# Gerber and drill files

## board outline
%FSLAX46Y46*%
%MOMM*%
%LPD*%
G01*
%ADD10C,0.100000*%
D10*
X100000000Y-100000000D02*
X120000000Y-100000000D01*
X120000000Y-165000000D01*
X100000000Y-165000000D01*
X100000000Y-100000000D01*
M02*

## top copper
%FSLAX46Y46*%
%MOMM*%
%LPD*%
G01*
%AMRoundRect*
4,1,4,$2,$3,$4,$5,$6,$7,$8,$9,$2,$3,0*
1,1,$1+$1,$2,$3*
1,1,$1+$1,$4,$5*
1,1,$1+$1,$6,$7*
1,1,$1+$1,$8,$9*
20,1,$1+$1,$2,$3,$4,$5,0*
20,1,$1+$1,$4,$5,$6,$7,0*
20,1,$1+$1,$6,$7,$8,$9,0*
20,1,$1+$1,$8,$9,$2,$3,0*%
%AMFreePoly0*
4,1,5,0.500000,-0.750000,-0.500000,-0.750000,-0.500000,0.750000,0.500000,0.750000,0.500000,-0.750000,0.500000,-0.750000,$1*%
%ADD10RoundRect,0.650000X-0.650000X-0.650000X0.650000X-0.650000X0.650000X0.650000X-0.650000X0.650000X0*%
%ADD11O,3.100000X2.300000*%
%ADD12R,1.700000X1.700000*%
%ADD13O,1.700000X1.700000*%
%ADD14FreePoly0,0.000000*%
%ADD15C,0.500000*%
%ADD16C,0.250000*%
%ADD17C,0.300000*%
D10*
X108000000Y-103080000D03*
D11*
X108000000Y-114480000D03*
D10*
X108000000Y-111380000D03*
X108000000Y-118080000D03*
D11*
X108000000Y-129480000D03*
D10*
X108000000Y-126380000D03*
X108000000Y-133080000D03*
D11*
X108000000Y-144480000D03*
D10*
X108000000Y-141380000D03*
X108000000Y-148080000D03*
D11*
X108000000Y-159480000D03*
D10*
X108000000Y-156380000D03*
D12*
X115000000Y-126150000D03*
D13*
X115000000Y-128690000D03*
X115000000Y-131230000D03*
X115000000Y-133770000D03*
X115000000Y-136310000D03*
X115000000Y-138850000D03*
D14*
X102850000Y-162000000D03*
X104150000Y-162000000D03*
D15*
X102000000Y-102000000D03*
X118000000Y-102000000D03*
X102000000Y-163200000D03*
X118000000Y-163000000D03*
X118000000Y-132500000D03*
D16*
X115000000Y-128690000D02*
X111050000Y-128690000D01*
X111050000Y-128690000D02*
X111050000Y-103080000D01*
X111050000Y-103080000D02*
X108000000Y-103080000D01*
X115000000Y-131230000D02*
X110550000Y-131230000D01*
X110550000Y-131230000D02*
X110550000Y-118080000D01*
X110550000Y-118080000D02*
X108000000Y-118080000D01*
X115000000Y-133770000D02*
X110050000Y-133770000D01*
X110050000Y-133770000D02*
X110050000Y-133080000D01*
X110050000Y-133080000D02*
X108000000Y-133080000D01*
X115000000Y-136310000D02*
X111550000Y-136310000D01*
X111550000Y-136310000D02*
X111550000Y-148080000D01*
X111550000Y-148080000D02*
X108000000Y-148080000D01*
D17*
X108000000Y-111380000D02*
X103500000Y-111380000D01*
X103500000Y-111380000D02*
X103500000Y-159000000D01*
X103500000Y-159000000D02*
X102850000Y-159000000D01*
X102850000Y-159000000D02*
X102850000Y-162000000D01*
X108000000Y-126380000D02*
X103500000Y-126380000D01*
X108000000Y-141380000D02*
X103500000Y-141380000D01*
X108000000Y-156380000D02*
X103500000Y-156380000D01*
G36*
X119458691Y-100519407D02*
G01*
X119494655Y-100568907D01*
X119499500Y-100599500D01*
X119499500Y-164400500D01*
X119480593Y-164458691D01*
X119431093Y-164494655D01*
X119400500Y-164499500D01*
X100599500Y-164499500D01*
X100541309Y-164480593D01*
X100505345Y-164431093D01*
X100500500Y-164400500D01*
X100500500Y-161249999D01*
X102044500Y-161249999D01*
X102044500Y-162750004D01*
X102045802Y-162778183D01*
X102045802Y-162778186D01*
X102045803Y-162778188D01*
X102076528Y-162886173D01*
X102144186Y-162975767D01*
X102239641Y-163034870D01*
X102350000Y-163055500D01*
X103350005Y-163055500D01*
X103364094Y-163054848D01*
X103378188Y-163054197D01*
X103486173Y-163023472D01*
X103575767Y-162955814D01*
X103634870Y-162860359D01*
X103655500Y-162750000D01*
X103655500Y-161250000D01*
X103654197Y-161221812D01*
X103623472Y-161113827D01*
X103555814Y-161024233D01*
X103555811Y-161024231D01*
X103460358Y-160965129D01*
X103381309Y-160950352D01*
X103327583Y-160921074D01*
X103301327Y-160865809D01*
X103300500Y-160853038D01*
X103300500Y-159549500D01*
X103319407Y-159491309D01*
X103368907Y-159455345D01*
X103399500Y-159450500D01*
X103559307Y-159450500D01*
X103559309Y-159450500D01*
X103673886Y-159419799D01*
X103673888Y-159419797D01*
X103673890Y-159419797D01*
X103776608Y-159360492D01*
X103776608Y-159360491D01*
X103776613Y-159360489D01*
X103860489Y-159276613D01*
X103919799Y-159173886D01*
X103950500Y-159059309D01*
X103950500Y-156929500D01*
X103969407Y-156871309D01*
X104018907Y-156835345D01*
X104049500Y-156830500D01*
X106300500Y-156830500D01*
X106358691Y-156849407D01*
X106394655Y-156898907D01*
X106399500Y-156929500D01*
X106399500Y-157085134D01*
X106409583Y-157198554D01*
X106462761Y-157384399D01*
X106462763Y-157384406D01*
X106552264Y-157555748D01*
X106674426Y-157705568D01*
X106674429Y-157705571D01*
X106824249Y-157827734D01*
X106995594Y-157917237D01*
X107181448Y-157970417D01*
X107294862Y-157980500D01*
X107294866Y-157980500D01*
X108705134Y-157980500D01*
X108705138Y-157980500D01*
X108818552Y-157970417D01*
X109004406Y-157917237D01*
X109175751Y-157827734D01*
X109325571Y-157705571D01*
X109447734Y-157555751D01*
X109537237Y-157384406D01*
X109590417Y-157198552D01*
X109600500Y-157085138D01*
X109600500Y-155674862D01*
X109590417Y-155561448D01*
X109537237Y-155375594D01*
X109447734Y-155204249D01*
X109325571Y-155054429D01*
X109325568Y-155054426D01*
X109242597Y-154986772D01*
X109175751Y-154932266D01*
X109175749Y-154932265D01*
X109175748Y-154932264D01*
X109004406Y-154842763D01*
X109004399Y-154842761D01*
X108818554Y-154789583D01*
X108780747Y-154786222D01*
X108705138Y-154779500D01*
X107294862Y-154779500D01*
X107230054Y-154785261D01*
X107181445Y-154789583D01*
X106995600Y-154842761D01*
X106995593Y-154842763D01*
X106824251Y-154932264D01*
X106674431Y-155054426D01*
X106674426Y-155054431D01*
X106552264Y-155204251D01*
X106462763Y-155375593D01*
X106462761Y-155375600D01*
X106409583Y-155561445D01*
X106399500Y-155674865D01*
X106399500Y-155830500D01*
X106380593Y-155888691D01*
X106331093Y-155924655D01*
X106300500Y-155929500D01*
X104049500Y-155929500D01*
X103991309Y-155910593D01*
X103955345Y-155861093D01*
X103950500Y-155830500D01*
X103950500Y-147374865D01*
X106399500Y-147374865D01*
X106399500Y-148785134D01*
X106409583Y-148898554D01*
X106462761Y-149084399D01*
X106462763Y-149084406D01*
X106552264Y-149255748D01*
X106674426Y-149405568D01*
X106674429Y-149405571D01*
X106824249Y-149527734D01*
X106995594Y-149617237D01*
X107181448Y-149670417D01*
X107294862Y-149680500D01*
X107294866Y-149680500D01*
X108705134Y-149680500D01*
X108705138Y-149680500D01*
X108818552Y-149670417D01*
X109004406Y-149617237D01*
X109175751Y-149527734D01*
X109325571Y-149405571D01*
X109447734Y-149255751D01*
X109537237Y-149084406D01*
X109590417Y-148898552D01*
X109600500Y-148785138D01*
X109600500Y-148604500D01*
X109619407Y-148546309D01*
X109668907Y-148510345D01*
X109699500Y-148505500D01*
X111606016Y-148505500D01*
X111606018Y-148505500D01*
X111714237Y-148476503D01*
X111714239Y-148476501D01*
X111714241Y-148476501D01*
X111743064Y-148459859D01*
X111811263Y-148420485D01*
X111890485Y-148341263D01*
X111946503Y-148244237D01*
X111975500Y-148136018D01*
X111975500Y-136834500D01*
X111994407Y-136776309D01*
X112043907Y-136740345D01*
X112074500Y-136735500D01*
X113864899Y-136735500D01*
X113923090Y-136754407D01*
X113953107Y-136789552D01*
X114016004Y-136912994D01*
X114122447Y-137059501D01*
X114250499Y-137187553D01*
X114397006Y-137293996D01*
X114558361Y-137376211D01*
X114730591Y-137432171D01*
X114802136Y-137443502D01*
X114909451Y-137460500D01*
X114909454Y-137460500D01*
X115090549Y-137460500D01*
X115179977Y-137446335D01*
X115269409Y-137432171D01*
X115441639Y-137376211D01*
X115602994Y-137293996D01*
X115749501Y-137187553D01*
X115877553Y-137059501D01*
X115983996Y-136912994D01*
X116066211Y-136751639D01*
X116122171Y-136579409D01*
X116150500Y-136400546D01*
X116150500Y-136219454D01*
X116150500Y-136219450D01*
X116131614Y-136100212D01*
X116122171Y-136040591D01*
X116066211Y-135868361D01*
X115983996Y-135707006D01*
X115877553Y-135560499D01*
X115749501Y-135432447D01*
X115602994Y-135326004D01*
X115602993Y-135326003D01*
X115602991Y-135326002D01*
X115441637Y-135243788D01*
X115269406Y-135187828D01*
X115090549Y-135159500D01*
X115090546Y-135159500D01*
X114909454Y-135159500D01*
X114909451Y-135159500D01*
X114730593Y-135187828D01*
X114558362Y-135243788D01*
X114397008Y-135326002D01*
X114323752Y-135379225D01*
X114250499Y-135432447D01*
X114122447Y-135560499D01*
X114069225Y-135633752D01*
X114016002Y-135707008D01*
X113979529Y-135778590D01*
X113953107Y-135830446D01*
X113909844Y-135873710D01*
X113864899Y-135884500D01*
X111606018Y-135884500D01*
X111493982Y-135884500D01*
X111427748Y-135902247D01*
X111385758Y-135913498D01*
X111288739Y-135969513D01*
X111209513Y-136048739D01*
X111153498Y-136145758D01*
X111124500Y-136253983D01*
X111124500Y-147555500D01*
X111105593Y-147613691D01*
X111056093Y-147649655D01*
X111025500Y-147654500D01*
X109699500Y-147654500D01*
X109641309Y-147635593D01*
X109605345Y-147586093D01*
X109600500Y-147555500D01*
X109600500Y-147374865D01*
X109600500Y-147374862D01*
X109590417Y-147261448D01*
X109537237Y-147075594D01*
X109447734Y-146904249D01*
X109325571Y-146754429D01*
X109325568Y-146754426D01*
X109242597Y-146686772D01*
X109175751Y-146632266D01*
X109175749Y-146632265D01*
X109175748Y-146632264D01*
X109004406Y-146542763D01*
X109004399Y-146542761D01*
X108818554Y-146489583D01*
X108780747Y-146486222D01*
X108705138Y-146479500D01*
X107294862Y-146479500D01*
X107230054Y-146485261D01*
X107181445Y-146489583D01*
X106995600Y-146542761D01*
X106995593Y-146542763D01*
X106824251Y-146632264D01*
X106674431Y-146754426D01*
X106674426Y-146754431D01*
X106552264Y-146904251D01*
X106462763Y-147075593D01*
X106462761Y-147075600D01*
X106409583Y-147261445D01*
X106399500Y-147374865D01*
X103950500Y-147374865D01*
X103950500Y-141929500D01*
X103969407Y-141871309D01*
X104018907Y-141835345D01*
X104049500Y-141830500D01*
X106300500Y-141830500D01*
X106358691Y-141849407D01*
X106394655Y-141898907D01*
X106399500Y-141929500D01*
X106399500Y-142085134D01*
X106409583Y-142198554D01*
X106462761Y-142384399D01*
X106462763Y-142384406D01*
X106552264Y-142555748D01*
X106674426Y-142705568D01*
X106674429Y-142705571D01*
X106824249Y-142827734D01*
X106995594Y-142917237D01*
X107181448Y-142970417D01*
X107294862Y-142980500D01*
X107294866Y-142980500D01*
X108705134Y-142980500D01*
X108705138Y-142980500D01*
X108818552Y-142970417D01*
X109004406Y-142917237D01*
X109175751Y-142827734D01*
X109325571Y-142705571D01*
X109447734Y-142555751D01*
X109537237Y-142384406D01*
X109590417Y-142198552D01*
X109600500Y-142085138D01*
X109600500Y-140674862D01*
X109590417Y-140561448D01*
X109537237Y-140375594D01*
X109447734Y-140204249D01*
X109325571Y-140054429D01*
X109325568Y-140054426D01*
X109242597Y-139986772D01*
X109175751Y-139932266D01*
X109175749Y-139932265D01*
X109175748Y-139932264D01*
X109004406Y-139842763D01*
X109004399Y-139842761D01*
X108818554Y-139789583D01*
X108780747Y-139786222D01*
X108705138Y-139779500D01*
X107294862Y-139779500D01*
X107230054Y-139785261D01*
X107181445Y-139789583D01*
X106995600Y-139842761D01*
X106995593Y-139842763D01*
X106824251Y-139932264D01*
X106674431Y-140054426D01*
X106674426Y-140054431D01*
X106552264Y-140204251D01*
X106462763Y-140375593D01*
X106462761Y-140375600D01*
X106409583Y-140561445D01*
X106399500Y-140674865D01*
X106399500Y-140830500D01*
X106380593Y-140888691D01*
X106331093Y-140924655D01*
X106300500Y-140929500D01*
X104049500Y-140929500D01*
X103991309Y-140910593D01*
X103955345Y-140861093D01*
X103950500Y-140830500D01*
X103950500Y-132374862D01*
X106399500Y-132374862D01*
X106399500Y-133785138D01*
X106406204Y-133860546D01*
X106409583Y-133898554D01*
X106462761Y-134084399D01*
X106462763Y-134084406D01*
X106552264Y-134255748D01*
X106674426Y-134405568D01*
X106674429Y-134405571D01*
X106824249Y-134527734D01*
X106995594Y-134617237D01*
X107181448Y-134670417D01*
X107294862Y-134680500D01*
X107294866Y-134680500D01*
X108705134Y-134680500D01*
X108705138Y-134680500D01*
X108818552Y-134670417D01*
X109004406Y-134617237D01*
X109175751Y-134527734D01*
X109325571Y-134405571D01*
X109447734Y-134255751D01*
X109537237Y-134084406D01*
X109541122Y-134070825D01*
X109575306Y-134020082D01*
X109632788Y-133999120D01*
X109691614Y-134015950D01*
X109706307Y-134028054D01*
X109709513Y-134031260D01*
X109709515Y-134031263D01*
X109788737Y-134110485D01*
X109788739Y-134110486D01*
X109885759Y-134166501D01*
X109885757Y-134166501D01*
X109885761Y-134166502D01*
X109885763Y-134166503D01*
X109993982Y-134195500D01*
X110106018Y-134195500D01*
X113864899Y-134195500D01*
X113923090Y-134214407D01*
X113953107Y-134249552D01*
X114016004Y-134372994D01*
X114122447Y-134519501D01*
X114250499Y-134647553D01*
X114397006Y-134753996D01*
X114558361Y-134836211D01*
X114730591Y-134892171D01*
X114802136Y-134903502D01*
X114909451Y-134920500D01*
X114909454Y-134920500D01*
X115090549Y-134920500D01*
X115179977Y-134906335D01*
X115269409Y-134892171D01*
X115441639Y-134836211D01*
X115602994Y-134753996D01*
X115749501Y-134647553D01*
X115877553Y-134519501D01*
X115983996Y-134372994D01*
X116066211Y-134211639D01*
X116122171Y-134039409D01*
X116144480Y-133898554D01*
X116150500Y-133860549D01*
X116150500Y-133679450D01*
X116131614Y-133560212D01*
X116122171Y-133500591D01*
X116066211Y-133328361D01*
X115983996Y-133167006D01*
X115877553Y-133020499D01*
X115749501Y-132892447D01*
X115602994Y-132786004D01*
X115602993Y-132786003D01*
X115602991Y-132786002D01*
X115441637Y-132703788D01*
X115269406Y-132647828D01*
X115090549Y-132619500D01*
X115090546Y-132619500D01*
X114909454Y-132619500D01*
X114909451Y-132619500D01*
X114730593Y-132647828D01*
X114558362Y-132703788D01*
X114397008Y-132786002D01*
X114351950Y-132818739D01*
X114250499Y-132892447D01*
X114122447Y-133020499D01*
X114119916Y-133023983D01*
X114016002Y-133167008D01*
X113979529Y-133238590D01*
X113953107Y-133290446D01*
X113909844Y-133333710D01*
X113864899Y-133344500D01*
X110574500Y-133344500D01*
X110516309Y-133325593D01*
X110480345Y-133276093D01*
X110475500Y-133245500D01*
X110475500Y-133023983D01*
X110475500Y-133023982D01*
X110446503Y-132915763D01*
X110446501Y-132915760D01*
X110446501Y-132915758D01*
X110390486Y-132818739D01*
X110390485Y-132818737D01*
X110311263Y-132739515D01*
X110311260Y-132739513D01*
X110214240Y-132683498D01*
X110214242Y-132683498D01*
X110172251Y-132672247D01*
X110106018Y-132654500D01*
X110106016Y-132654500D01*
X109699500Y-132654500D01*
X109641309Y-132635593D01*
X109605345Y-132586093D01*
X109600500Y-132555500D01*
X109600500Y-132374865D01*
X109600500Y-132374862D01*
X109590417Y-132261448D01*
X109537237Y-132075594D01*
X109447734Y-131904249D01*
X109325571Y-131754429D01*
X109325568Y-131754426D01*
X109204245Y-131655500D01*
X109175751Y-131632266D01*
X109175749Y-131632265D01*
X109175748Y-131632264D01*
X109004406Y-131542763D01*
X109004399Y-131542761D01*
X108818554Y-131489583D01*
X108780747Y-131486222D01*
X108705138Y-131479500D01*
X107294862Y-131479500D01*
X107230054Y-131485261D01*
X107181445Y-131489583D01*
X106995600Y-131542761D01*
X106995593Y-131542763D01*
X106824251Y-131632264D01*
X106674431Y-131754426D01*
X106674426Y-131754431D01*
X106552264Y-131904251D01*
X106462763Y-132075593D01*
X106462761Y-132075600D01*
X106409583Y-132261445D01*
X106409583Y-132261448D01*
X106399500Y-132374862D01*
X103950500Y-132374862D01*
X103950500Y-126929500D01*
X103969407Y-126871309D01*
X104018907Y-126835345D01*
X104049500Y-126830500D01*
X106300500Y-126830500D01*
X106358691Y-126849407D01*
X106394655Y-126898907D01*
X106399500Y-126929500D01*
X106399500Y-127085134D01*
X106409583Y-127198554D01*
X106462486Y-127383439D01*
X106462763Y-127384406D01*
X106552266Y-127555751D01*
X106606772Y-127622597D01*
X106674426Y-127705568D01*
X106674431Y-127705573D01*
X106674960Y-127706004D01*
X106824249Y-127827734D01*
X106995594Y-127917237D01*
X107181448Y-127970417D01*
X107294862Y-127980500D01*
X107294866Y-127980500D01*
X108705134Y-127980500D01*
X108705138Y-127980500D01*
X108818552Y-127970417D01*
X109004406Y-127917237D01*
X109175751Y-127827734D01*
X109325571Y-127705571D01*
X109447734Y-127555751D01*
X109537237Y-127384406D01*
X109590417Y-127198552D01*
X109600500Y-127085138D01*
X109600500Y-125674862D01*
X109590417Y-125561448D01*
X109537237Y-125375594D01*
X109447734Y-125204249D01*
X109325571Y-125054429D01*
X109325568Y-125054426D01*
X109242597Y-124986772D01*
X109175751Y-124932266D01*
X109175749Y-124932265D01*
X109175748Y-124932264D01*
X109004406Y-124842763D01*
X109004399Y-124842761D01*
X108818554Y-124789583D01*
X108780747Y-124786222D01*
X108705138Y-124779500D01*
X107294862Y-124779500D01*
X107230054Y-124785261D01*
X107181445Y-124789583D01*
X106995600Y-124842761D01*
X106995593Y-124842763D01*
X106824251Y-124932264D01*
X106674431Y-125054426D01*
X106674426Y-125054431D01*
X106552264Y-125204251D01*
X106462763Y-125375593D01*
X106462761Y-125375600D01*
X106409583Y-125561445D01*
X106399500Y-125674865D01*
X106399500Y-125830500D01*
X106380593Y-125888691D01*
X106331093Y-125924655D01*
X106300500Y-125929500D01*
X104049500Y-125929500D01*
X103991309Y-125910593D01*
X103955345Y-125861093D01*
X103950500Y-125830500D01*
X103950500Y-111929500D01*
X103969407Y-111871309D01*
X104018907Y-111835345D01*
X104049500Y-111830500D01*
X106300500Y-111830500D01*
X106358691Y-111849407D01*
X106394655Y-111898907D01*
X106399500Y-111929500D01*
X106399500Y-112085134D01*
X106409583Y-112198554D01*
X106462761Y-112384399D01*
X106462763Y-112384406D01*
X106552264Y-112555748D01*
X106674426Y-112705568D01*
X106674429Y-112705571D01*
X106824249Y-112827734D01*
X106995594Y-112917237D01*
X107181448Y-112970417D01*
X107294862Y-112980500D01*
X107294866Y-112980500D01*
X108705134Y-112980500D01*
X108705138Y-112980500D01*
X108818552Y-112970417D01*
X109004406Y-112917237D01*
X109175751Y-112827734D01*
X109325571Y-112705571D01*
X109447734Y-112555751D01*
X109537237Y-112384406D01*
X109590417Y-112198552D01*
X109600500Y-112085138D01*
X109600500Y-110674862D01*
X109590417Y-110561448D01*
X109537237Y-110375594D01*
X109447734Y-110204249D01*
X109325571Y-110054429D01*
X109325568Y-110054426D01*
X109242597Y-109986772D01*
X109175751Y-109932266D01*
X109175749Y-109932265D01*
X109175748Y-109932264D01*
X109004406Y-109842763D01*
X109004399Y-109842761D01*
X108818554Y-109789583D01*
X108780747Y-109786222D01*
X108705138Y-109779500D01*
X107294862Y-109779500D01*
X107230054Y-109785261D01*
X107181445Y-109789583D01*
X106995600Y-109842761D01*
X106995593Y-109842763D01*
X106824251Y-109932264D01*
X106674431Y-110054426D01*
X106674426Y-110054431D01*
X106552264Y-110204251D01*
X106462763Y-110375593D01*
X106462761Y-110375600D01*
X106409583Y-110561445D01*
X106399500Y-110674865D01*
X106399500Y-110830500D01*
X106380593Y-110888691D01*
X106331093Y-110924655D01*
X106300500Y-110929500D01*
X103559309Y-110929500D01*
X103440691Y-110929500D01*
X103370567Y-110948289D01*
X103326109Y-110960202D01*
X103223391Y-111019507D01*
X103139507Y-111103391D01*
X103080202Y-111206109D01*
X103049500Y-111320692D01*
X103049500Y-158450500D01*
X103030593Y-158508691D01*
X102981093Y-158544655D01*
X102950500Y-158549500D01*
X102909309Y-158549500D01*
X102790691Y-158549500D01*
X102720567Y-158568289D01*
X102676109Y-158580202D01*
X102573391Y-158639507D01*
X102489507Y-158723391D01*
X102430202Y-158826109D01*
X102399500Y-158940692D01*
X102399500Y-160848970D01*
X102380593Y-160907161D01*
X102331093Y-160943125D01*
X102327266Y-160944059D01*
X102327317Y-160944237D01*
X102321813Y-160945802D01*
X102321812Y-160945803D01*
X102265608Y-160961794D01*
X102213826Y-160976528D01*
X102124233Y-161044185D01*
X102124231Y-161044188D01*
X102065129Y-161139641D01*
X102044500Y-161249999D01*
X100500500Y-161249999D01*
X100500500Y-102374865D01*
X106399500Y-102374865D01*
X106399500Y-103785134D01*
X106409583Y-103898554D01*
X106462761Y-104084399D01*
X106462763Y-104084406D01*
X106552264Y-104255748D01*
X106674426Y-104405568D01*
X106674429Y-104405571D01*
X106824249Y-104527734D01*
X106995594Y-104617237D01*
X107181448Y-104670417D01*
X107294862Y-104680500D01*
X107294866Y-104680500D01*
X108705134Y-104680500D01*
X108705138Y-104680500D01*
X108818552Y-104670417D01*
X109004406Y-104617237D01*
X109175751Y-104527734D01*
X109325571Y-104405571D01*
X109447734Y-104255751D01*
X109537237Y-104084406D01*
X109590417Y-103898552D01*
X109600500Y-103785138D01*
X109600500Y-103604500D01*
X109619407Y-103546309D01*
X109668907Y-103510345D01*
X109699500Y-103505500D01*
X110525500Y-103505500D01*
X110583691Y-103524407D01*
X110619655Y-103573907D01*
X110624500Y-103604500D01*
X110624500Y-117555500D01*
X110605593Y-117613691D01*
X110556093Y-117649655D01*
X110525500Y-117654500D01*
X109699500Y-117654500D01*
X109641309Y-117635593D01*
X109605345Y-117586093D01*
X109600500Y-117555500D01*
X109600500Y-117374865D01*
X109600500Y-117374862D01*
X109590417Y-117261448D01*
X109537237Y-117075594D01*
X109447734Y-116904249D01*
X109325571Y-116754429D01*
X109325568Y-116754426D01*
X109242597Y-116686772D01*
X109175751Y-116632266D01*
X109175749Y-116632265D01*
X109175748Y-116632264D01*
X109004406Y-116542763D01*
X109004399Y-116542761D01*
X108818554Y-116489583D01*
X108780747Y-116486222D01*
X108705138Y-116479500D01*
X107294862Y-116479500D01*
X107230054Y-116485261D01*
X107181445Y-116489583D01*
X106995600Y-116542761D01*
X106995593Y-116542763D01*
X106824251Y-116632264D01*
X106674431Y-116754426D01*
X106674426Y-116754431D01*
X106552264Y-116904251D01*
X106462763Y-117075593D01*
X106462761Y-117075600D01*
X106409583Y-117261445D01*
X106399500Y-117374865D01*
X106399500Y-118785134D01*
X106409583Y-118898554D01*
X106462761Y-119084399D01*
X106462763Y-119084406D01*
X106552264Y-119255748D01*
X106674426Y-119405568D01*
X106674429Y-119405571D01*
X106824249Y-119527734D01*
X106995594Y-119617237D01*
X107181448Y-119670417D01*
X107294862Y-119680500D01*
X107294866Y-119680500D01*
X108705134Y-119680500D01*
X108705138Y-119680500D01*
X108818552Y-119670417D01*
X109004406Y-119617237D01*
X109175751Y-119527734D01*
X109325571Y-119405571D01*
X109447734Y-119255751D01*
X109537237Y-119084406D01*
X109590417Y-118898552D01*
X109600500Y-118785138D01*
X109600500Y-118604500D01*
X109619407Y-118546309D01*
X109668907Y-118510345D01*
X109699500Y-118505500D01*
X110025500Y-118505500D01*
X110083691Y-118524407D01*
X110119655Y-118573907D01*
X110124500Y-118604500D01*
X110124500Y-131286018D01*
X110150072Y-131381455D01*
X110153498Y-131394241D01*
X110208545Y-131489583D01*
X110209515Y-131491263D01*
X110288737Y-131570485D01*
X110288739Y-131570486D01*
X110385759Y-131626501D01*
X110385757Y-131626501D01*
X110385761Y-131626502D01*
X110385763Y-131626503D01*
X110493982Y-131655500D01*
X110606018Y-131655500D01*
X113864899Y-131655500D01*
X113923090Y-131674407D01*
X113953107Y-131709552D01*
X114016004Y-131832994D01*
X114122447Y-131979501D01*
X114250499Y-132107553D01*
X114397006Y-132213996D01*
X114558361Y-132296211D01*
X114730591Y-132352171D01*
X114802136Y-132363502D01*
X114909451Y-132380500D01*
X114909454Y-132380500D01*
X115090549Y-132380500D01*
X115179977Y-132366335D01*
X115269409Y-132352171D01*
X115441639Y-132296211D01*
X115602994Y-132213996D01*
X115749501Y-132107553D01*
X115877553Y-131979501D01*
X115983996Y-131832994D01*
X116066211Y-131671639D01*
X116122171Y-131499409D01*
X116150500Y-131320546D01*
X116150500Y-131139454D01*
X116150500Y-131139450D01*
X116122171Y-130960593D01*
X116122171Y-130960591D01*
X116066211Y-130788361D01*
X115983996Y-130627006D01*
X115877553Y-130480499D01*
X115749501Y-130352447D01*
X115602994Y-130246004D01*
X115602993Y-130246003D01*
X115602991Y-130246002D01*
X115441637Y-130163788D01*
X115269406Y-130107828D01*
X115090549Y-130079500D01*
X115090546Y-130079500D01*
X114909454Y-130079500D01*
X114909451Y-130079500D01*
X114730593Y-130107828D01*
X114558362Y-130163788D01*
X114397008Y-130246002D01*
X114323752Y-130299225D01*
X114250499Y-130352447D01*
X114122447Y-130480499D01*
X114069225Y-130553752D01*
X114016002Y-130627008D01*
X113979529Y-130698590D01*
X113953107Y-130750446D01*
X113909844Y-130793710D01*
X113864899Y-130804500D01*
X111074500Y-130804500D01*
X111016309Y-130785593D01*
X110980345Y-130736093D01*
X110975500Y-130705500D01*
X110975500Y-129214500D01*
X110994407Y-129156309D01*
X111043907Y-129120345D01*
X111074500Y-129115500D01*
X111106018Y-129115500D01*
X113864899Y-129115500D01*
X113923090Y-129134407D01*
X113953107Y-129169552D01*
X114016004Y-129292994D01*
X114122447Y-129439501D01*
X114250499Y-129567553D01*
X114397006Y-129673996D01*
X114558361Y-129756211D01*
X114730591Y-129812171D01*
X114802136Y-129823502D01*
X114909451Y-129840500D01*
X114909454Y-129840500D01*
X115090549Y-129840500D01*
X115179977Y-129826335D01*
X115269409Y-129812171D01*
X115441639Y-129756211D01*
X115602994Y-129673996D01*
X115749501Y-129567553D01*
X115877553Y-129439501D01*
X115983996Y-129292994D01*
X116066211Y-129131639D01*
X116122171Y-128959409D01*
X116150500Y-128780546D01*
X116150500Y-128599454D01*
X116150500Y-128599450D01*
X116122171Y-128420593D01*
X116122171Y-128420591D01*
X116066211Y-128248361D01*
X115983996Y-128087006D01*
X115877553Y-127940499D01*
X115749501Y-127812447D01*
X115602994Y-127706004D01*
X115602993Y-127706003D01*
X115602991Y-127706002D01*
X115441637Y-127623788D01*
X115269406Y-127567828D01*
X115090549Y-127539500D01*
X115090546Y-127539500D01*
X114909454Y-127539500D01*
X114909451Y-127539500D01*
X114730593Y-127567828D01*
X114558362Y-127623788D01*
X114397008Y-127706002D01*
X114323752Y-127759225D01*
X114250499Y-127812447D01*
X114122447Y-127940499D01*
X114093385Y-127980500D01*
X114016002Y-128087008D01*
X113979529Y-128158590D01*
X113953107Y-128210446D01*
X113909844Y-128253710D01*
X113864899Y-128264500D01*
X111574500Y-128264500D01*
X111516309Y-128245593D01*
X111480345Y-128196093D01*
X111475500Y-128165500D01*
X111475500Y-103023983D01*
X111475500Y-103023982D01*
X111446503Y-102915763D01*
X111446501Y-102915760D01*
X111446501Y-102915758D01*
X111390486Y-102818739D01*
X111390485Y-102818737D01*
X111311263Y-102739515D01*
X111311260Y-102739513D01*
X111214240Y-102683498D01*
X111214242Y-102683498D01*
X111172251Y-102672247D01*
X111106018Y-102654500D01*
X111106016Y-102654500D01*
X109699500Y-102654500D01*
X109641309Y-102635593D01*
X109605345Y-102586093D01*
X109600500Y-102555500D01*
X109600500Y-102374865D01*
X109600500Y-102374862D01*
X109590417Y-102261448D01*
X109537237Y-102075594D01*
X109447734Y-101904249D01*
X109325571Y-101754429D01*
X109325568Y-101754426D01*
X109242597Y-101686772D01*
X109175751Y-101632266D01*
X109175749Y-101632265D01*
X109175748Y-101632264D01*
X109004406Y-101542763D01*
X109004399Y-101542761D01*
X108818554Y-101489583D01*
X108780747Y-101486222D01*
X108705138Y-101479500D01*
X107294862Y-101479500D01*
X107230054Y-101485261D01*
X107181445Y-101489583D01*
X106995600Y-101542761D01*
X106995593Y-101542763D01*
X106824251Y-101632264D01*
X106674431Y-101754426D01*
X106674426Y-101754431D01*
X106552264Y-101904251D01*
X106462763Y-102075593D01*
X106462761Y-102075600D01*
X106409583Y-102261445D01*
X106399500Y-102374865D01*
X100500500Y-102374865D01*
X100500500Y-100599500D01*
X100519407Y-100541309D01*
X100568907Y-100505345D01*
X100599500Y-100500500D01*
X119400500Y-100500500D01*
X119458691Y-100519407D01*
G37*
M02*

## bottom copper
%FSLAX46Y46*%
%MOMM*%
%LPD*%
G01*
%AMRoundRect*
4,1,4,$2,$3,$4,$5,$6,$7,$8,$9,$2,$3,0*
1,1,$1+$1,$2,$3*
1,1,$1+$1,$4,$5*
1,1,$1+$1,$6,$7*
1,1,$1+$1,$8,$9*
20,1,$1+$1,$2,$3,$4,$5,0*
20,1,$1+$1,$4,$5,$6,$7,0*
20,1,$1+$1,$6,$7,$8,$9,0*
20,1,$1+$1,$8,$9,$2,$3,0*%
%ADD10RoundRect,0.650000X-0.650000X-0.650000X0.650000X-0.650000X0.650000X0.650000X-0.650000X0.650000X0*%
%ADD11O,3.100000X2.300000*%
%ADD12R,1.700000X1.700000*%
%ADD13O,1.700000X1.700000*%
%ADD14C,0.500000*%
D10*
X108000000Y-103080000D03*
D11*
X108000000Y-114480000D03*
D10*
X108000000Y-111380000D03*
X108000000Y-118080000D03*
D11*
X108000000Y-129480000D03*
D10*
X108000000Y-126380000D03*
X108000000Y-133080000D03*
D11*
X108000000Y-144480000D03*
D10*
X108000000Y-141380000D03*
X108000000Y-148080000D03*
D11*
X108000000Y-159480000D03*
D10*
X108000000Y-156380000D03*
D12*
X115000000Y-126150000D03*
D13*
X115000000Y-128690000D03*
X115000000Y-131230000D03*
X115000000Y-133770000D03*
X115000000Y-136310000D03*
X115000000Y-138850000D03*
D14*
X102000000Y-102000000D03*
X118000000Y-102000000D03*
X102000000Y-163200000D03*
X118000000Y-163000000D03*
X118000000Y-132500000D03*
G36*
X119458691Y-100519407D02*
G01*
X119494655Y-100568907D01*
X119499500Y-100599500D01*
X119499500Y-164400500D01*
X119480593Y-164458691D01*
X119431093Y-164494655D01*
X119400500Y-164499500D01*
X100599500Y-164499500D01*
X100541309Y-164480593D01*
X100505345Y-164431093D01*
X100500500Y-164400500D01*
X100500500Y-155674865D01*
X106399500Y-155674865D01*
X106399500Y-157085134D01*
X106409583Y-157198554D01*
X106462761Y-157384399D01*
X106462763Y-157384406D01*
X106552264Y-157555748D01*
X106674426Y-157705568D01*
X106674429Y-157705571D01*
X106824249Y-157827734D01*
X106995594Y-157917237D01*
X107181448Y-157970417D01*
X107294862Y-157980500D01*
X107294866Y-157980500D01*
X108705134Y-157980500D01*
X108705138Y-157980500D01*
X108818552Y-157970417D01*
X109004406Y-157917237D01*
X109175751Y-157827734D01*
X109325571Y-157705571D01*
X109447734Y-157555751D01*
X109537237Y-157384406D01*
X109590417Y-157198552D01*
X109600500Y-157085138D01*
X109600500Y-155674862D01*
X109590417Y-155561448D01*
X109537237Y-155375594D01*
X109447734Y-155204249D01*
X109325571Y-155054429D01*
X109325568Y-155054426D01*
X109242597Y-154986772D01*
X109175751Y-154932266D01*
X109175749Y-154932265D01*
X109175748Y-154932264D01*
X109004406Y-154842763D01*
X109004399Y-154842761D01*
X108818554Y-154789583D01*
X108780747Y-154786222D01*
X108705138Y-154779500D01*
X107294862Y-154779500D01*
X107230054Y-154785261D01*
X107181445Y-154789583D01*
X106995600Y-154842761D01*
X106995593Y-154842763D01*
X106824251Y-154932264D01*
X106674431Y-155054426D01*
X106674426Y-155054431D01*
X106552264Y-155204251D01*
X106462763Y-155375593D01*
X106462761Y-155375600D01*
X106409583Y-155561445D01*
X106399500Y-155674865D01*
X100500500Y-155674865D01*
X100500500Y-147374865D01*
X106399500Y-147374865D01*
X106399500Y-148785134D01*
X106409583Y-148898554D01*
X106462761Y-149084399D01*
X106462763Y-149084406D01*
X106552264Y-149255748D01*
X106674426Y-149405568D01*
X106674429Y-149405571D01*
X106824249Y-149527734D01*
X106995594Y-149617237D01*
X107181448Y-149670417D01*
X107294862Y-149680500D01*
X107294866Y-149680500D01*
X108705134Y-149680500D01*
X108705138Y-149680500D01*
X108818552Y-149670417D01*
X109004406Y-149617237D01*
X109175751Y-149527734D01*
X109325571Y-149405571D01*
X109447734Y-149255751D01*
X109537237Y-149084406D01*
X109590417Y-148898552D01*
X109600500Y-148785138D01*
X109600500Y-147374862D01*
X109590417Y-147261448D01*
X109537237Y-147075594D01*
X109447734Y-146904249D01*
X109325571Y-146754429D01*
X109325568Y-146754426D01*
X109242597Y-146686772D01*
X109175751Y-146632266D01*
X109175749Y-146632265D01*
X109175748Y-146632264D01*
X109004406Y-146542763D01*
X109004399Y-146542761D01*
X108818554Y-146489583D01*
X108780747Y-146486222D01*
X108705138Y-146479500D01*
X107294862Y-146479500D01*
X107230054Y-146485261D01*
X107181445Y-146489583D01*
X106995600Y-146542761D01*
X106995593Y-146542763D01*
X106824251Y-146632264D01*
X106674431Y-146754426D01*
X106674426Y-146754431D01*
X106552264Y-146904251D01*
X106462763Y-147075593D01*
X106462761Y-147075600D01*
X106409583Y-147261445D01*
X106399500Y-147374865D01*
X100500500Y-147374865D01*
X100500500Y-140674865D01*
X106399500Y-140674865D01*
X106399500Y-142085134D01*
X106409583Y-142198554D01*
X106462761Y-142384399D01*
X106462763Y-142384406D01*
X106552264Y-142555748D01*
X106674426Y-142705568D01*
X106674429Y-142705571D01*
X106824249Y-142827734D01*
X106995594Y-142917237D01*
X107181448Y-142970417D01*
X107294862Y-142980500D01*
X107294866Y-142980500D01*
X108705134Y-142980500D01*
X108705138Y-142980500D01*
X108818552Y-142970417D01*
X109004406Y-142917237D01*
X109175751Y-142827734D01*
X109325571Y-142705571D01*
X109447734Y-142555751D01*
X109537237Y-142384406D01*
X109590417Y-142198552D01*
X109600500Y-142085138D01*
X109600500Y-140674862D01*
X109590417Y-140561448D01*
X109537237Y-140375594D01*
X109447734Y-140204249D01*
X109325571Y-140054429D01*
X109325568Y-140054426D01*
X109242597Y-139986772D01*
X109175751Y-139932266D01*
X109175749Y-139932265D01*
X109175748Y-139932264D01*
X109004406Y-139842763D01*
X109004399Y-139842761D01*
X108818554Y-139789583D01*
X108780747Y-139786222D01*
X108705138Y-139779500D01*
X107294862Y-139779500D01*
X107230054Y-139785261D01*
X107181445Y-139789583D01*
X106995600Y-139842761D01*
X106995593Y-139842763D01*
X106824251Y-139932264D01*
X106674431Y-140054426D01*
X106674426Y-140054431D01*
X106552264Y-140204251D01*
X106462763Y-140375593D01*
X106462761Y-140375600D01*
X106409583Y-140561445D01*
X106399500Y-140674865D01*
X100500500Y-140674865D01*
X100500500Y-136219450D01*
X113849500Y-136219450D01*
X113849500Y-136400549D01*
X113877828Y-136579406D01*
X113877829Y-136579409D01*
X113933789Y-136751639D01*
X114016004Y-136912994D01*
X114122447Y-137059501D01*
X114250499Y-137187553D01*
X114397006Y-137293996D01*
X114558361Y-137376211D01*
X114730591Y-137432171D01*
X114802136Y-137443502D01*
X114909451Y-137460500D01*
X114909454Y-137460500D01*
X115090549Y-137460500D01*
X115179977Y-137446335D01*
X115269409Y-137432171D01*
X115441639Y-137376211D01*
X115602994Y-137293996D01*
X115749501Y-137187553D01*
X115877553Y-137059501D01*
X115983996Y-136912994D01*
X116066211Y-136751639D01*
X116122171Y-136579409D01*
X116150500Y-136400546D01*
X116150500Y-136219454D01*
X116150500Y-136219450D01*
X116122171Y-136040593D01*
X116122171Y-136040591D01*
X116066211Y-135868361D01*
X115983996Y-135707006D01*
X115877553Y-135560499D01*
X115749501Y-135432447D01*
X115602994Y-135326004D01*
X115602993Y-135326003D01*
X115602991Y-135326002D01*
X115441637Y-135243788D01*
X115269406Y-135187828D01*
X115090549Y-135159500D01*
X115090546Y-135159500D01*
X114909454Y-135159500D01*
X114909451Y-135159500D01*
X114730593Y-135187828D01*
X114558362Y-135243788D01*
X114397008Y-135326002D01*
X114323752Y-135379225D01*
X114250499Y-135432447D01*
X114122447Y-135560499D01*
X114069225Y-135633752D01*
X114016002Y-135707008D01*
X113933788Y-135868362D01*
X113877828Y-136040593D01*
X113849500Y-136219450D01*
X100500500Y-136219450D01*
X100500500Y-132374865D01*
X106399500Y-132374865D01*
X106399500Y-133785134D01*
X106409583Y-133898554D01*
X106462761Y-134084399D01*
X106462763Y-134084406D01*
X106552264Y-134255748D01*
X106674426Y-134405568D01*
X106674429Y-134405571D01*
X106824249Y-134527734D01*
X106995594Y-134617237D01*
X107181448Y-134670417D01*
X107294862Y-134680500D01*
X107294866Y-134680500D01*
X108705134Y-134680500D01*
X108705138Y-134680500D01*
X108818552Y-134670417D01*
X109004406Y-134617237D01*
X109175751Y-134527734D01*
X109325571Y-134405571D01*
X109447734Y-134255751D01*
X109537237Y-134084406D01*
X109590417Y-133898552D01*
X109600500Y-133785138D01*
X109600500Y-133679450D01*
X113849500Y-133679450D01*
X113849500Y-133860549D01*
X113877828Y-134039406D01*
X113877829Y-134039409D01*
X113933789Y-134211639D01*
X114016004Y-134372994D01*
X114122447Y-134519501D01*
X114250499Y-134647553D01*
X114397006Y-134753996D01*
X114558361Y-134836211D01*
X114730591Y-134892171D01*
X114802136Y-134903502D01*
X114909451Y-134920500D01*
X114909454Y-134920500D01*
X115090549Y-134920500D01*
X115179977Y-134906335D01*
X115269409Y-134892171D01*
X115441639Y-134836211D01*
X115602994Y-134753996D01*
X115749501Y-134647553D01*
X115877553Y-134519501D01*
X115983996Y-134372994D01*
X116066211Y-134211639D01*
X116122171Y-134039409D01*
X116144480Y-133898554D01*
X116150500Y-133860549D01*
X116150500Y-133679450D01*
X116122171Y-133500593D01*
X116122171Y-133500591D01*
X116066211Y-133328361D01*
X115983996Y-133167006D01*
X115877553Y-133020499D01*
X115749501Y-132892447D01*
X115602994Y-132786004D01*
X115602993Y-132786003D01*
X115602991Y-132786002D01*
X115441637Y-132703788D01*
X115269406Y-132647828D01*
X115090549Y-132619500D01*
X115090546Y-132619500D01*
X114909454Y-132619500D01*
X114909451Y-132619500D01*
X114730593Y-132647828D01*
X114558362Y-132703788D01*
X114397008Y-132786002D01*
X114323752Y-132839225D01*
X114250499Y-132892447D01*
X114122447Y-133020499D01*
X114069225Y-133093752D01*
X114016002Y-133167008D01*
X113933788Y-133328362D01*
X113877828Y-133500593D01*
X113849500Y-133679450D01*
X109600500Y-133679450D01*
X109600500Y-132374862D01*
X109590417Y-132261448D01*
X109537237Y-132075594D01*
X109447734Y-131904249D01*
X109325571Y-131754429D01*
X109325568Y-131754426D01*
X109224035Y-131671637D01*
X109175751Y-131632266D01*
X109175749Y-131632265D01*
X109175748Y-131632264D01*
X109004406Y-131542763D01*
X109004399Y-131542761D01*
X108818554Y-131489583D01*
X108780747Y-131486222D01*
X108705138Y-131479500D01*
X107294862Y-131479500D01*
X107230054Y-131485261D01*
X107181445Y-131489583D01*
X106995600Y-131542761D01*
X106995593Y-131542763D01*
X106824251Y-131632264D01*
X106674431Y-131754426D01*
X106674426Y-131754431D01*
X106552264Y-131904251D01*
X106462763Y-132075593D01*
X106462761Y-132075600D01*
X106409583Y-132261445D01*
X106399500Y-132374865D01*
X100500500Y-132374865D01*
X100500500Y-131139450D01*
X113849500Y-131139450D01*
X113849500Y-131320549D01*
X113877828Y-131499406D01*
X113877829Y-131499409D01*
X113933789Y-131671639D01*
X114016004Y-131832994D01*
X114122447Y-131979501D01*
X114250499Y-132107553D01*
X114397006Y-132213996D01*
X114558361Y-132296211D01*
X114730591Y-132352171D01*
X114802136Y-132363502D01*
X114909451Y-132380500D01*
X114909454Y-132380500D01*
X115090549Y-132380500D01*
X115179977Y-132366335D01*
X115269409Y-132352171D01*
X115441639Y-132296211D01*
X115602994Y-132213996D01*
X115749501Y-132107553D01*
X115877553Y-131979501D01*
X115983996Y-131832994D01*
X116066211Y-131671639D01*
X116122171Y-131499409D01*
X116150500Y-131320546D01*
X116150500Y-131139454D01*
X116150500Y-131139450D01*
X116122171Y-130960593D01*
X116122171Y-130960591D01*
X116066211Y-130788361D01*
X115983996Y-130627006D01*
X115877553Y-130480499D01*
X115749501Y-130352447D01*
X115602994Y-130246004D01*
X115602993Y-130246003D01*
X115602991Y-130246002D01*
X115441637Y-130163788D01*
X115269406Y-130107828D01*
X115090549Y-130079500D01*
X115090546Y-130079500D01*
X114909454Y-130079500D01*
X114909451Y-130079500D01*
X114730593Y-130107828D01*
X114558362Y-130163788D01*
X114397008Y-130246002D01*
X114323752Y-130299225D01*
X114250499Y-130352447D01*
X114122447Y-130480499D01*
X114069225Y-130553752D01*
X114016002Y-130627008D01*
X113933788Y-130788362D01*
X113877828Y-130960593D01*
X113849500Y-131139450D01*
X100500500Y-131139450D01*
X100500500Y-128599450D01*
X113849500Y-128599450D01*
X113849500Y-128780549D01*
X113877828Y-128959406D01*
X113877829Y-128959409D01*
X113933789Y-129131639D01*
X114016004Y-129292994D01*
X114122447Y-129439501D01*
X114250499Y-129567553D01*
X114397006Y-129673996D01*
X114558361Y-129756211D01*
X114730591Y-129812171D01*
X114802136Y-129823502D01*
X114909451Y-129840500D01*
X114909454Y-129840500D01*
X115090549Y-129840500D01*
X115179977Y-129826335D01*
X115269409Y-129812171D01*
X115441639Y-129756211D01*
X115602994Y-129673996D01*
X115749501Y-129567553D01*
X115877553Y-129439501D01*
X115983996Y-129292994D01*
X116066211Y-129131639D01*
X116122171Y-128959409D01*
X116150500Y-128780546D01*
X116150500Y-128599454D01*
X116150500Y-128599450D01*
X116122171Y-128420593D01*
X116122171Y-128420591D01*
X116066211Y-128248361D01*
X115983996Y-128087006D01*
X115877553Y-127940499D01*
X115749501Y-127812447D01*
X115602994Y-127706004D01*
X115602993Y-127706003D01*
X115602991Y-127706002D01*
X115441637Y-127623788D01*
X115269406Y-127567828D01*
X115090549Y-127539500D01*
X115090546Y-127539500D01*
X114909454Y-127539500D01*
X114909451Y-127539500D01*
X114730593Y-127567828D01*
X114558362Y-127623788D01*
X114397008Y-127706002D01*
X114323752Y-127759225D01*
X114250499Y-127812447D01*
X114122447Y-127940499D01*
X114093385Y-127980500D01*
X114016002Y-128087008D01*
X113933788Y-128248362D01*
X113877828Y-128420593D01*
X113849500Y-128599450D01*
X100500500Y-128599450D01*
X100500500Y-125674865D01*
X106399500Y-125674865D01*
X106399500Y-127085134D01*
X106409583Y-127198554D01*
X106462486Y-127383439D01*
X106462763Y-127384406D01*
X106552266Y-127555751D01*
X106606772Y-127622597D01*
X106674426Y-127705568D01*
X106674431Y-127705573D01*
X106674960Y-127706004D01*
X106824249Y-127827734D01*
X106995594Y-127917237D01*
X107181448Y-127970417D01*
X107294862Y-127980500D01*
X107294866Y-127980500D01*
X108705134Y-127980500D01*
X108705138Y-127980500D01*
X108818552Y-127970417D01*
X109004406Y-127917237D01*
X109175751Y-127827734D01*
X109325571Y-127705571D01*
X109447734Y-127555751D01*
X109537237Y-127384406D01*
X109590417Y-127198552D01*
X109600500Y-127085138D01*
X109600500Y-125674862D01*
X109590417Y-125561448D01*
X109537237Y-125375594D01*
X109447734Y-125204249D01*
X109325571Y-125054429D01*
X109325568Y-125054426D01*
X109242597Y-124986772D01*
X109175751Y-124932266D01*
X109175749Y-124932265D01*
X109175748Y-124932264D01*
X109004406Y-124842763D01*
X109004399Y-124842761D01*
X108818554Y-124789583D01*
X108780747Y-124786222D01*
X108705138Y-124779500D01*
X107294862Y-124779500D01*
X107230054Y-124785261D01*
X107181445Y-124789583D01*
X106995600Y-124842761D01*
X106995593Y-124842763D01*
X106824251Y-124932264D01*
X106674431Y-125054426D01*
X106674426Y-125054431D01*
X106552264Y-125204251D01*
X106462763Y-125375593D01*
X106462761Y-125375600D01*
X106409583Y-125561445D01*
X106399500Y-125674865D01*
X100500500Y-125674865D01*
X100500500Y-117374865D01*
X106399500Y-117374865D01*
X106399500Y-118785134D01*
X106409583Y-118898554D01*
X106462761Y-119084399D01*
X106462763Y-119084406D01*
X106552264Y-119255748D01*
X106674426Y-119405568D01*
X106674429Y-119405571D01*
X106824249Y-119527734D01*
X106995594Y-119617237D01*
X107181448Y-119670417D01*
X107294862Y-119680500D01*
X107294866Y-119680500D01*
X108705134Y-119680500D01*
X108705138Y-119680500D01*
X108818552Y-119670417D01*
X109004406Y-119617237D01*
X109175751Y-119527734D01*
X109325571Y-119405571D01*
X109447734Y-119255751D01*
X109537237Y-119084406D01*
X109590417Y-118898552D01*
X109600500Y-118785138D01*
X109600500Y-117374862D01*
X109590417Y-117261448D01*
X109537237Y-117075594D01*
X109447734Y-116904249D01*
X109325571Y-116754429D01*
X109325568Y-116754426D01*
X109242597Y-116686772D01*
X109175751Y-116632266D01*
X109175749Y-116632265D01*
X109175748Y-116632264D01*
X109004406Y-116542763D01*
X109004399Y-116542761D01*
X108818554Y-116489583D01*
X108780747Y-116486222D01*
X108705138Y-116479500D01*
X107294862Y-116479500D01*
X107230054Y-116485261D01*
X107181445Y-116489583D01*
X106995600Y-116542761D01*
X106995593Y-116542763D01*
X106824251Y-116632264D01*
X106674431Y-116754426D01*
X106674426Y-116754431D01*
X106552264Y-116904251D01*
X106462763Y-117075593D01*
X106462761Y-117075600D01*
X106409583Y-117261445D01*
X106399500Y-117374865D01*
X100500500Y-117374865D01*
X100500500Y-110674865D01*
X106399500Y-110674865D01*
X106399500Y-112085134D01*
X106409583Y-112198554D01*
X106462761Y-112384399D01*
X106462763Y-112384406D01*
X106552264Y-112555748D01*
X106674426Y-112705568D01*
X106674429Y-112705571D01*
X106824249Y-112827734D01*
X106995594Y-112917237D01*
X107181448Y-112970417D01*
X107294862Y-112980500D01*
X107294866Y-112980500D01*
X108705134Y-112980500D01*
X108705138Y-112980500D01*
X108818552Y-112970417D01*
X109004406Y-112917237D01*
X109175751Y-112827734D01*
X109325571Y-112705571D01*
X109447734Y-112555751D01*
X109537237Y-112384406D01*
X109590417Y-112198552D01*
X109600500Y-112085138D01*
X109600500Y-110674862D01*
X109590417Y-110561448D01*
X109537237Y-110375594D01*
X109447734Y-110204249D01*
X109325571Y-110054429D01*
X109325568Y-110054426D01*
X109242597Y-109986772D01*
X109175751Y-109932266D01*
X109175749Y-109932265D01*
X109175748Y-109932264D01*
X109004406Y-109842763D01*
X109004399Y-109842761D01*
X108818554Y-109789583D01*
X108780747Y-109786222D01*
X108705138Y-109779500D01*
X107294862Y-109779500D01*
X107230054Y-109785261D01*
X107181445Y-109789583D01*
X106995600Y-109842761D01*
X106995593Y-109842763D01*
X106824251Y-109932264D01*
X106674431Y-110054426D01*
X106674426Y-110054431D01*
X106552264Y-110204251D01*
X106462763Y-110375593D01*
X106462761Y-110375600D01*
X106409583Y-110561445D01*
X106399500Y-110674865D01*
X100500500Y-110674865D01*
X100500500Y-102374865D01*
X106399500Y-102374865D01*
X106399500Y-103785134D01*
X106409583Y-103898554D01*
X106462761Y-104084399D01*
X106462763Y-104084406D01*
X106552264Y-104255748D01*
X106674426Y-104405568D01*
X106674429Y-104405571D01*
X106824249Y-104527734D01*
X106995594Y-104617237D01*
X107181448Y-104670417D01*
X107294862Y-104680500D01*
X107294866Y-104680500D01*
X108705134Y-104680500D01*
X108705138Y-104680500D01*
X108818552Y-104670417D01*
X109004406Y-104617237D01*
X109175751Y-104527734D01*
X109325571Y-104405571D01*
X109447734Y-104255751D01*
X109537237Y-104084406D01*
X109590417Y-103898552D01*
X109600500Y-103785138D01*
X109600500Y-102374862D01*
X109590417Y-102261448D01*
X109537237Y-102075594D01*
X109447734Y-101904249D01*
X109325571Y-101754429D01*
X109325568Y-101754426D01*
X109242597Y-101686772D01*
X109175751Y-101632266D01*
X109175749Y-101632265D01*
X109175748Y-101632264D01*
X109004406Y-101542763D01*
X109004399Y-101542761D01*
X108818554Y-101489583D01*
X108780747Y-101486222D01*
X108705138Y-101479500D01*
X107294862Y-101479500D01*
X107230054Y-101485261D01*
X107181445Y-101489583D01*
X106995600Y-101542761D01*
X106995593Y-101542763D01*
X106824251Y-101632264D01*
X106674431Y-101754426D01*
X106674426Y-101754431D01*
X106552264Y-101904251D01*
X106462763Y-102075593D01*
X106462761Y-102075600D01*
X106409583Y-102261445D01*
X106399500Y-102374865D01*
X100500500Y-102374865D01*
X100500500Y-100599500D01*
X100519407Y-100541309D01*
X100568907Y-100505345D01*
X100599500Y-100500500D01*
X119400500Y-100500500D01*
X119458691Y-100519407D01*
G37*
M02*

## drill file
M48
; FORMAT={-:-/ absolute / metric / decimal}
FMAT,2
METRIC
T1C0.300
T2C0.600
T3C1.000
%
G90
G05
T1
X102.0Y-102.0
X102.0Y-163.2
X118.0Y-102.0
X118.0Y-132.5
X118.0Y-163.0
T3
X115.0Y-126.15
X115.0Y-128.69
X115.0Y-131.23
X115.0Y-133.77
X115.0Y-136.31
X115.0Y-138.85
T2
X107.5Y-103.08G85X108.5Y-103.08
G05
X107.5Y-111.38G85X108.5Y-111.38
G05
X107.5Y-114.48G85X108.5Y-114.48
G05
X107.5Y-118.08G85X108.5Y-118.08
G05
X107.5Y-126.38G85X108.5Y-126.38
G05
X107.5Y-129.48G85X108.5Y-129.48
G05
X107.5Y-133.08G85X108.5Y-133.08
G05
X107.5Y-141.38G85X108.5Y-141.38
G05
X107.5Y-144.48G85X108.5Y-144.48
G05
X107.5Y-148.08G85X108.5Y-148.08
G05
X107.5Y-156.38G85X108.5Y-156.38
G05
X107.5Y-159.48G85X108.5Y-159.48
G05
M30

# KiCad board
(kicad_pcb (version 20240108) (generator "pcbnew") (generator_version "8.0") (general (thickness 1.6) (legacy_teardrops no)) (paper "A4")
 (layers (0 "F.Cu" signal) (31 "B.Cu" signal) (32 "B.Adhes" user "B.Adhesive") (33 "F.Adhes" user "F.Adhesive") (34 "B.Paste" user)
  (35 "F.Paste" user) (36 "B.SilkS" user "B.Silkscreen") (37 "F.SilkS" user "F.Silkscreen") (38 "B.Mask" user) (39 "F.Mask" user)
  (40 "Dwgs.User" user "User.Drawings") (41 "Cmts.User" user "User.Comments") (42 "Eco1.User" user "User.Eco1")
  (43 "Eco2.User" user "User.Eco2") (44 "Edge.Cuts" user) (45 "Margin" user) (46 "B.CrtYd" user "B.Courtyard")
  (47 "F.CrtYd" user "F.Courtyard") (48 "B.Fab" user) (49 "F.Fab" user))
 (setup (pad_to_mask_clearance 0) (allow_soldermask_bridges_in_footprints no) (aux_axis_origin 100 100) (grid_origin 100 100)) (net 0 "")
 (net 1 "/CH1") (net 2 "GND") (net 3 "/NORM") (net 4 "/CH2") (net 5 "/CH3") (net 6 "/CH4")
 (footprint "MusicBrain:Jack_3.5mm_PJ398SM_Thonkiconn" (layer "F.Cu") (at 108 108)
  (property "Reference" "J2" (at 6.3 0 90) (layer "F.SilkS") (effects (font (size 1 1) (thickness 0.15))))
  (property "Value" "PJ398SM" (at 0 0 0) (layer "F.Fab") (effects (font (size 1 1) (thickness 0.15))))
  (pad "1" thru_hole roundrect (at 0 -4.92) (size 2.6 2.6) (drill oval 1.6 0.6) (layers "*.Cu" "*.Mask") (roundrect_rratio 0.25)
   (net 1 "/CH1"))
  (pad "2" thru_hole oval (at 0 6.48) (size 3.1 2.3) (drill oval 1.6 0.6) (layers "*.Cu" "*.Mask") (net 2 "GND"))
  (pad "3" thru_hole roundrect (at 0 3.38) (size 2.6 2.6) (drill oval 1.6 0.6) (layers "*.Cu" "*.Mask") (roundrect_rratio 0.25)
   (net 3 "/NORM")))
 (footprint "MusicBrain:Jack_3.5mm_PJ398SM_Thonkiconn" (layer "F.Cu") (at 108 123)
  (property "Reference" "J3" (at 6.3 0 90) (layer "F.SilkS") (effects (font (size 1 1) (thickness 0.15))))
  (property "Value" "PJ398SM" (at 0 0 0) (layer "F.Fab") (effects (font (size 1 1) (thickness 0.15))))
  (pad "1" thru_hole roundrect (at 0 -4.92) (size 2.6 2.6) (drill oval 1.6 0.6) (layers "*.Cu" "*.Mask") (roundrect_rratio 0.25)
   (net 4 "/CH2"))
  (pad "2" thru_hole oval (at 0 6.48) (size 3.1 2.3) (drill oval 1.6 0.6) (layers "*.Cu" "*.Mask") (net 2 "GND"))
  (pad "3" thru_hole roundrect (at 0 3.38) (size 2.6 2.6) (drill oval 1.6 0.6) (layers "*.Cu" "*.Mask") (roundrect_rratio 0.25)
   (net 3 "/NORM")))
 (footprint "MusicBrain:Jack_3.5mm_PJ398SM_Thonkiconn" (layer "F.Cu") (at 108 138)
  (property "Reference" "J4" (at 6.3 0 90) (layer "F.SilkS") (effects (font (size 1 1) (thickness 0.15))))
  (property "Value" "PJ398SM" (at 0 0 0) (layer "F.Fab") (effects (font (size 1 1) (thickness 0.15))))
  (pad "1" thru_hole roundrect (at 0 -4.92) (size 2.6 2.6) (drill oval 1.6 0.6) (layers "*.Cu" "*.Mask") (roundrect_rratio 0.25)
   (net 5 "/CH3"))
  (pad "2" thru_hole oval (at 0 6.48) (size 3.1 2.3) (drill oval 1.6 0.6) (layers "*.Cu" "*.Mask") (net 2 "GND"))
  (pad "3" thru_hole roundrect (at 0 3.38) (size 2.6 2.6) (drill oval 1.6 0.6) (layers "*.Cu" "*.Mask") (roundrect_rratio 0.25)
   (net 3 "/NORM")))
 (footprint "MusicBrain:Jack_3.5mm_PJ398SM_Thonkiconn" (layer "F.Cu") (at 108 153)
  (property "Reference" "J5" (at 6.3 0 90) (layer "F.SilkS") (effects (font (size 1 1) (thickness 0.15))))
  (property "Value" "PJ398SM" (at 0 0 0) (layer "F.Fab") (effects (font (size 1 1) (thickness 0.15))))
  (pad "1" thru_hole roundrect (at 0 -4.92) (size 2.6 2.6) (drill oval 1.6 0.6) (layers "*.Cu" "*.Mask") (roundrect_rratio 0.25)
   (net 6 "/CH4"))
  (pad "2" thru_hole oval (at 0 6.48) (size 3.1 2.3) (drill oval 1.6 0.6) (layers "*.Cu" "*.Mask") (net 2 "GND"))
  (pad "3" thru_hole roundrect (at 0 3.38) (size 2.6 2.6) (drill oval 1.6 0.6) (layers "*.Cu" "*.Mask") (roundrect_rratio 0.25)
   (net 3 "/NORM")))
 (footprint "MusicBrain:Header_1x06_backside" (layer "B.Cu") (at 115 126.15)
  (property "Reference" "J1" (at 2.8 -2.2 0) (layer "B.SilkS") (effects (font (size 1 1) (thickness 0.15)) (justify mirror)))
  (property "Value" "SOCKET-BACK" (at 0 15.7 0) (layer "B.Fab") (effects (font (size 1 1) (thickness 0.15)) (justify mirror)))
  (pad "1" thru_hole rect (at 0 0) (size 1.7 1.7) (drill 1.0) (layers "*.Cu" "*.Mask") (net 2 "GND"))
  (pad "2" thru_hole oval (at 0 2.54) (size 1.7 1.7) (drill 1.0) (layers "*.Cu" "*.Mask") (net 1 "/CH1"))
  (pad "3" thru_hole oval (at 0 5.08) (size 1.7 1.7) (drill 1.0) (layers "*.Cu" "*.Mask") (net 4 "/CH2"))
  (pad "4" thru_hole oval (at 0 7.62) (size 1.7 1.7) (drill 1.0) (layers "*.Cu" "*.Mask") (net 5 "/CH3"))
  (pad "5" thru_hole oval (at 0 10.16) (size 1.7 1.7) (drill 1.0) (layers "*.Cu" "*.Mask") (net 6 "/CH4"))
  (pad "6" thru_hole oval (at 0 12.7) (size 1.7 1.7) (drill 1.0) (layers "*.Cu" "*.Mask") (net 2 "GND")))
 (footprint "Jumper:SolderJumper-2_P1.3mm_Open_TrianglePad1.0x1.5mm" (layer "F.Cu") (at 103.5 162)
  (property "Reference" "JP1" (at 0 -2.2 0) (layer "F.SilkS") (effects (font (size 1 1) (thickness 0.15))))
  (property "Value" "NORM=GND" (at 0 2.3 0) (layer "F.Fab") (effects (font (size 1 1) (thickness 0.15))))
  (pad "1" smd custom (at -0.65 0) (size 1 1.5) (layers "F.Cu" "F.Mask") (options (clearance outline) (anchor rect)) (primitives)
   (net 3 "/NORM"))
  (pad "2" smd custom (at 0.65 0) (size 1 1.5) (layers "F.Cu" "F.Mask") (options (clearance outline) (anchor rect)) (primitives)
   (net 2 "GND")))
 (segment (start 115 128.69) (end 111.05 128.69) (width 0.25) (layer "F.Cu") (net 1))
 (segment (start 111.05 128.69) (end 111.05 103.08) (width 0.25) (layer "F.Cu") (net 1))
 (segment (start 111.05 103.08) (end 108 103.08) (width 0.25) (layer "F.Cu") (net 1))
 (segment (start 115 131.23) (end 110.55 131.23) (width 0.25) (layer "F.Cu") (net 4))
 (segment (start 110.55 131.23) (end 110.55 118.08) (width 0.25) (layer "F.Cu") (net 4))
 (segment (start 110.55 118.08) (end 108 118.08) (width 0.25) (layer "F.Cu") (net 4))
 (segment (start 115 133.77) (end 110.05 133.77) (width 0.25) (layer "F.Cu") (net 5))
 (segment (start 110.05 133.77) (end 110.05 133.08) (width 0.25) (layer "F.Cu") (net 5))
 (segment (start 110.05 133.08) (end 108 133.08) (width 0.25) (layer "F.Cu") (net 5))
 (segment (start 115 136.31) (end 111.55 136.31) (width 0.25) (layer "F.Cu") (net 6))
 (segment (start 111.55 136.31) (end 111.55 148.08) (width 0.25) (layer "F.Cu") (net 6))
 (segment (start 111.55 148.08) (end 108 148.08) (width 0.25) (layer "F.Cu") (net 6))
 (segment (start 108 111.38) (end 103.5 111.38) (width 0.3) (layer "F.Cu") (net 3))
 (segment (start 103.5 111.38) (end 103.5 159) (width 0.3) (layer "F.Cu") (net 3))
 (segment (start 103.5 159) (end 102.85 159) (width 0.3) (layer "F.Cu") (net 3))
 (segment (start 102.85 159) (end 102.85 162) (width 0.3) (layer "F.Cu") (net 3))
 (segment (start 108 126.38) (end 103.5 126.38) (width 0.3) (layer "F.Cu") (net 3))
 (segment (start 108 141.38) (end 103.5 141.38) (width 0.3) (layer "F.Cu") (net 3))
 (segment (start 108 156.38) (end 103.5 156.38) (width 0.3) (layer "F.Cu") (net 3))
 (via (at 102 102) (size 0.5) (drill 0.3) (layers "F.Cu" "B.Cu") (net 2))
 (via (at 118 102) (size 0.5) (drill 0.3) (layers "F.Cu" "B.Cu") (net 2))
 (via (at 102 163.2) (size 0.5) (drill 0.3) (layers "F.Cu" "B.Cu") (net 2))
 (via (at 118 163) (size 0.5) (drill 0.3) (layers "F.Cu" "B.Cu") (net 2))
 (via (at 118 132.5) (size 0.5) (drill 0.3) (layers "F.Cu" "B.Cu") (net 2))
 (gr_rect (start 100 100) (end 120 165) (stroke (width 0.1) (type default)) (fill none) (layer "Edge.Cuts"))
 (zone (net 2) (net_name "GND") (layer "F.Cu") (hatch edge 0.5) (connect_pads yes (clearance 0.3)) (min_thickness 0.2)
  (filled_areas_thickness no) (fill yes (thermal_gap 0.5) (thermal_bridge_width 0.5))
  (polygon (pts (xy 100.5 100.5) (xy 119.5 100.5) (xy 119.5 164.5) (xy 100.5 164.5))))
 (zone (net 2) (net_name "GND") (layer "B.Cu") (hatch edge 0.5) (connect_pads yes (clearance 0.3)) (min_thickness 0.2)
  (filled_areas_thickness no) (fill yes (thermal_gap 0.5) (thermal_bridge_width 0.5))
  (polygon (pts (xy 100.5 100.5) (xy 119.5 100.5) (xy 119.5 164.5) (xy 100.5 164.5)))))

